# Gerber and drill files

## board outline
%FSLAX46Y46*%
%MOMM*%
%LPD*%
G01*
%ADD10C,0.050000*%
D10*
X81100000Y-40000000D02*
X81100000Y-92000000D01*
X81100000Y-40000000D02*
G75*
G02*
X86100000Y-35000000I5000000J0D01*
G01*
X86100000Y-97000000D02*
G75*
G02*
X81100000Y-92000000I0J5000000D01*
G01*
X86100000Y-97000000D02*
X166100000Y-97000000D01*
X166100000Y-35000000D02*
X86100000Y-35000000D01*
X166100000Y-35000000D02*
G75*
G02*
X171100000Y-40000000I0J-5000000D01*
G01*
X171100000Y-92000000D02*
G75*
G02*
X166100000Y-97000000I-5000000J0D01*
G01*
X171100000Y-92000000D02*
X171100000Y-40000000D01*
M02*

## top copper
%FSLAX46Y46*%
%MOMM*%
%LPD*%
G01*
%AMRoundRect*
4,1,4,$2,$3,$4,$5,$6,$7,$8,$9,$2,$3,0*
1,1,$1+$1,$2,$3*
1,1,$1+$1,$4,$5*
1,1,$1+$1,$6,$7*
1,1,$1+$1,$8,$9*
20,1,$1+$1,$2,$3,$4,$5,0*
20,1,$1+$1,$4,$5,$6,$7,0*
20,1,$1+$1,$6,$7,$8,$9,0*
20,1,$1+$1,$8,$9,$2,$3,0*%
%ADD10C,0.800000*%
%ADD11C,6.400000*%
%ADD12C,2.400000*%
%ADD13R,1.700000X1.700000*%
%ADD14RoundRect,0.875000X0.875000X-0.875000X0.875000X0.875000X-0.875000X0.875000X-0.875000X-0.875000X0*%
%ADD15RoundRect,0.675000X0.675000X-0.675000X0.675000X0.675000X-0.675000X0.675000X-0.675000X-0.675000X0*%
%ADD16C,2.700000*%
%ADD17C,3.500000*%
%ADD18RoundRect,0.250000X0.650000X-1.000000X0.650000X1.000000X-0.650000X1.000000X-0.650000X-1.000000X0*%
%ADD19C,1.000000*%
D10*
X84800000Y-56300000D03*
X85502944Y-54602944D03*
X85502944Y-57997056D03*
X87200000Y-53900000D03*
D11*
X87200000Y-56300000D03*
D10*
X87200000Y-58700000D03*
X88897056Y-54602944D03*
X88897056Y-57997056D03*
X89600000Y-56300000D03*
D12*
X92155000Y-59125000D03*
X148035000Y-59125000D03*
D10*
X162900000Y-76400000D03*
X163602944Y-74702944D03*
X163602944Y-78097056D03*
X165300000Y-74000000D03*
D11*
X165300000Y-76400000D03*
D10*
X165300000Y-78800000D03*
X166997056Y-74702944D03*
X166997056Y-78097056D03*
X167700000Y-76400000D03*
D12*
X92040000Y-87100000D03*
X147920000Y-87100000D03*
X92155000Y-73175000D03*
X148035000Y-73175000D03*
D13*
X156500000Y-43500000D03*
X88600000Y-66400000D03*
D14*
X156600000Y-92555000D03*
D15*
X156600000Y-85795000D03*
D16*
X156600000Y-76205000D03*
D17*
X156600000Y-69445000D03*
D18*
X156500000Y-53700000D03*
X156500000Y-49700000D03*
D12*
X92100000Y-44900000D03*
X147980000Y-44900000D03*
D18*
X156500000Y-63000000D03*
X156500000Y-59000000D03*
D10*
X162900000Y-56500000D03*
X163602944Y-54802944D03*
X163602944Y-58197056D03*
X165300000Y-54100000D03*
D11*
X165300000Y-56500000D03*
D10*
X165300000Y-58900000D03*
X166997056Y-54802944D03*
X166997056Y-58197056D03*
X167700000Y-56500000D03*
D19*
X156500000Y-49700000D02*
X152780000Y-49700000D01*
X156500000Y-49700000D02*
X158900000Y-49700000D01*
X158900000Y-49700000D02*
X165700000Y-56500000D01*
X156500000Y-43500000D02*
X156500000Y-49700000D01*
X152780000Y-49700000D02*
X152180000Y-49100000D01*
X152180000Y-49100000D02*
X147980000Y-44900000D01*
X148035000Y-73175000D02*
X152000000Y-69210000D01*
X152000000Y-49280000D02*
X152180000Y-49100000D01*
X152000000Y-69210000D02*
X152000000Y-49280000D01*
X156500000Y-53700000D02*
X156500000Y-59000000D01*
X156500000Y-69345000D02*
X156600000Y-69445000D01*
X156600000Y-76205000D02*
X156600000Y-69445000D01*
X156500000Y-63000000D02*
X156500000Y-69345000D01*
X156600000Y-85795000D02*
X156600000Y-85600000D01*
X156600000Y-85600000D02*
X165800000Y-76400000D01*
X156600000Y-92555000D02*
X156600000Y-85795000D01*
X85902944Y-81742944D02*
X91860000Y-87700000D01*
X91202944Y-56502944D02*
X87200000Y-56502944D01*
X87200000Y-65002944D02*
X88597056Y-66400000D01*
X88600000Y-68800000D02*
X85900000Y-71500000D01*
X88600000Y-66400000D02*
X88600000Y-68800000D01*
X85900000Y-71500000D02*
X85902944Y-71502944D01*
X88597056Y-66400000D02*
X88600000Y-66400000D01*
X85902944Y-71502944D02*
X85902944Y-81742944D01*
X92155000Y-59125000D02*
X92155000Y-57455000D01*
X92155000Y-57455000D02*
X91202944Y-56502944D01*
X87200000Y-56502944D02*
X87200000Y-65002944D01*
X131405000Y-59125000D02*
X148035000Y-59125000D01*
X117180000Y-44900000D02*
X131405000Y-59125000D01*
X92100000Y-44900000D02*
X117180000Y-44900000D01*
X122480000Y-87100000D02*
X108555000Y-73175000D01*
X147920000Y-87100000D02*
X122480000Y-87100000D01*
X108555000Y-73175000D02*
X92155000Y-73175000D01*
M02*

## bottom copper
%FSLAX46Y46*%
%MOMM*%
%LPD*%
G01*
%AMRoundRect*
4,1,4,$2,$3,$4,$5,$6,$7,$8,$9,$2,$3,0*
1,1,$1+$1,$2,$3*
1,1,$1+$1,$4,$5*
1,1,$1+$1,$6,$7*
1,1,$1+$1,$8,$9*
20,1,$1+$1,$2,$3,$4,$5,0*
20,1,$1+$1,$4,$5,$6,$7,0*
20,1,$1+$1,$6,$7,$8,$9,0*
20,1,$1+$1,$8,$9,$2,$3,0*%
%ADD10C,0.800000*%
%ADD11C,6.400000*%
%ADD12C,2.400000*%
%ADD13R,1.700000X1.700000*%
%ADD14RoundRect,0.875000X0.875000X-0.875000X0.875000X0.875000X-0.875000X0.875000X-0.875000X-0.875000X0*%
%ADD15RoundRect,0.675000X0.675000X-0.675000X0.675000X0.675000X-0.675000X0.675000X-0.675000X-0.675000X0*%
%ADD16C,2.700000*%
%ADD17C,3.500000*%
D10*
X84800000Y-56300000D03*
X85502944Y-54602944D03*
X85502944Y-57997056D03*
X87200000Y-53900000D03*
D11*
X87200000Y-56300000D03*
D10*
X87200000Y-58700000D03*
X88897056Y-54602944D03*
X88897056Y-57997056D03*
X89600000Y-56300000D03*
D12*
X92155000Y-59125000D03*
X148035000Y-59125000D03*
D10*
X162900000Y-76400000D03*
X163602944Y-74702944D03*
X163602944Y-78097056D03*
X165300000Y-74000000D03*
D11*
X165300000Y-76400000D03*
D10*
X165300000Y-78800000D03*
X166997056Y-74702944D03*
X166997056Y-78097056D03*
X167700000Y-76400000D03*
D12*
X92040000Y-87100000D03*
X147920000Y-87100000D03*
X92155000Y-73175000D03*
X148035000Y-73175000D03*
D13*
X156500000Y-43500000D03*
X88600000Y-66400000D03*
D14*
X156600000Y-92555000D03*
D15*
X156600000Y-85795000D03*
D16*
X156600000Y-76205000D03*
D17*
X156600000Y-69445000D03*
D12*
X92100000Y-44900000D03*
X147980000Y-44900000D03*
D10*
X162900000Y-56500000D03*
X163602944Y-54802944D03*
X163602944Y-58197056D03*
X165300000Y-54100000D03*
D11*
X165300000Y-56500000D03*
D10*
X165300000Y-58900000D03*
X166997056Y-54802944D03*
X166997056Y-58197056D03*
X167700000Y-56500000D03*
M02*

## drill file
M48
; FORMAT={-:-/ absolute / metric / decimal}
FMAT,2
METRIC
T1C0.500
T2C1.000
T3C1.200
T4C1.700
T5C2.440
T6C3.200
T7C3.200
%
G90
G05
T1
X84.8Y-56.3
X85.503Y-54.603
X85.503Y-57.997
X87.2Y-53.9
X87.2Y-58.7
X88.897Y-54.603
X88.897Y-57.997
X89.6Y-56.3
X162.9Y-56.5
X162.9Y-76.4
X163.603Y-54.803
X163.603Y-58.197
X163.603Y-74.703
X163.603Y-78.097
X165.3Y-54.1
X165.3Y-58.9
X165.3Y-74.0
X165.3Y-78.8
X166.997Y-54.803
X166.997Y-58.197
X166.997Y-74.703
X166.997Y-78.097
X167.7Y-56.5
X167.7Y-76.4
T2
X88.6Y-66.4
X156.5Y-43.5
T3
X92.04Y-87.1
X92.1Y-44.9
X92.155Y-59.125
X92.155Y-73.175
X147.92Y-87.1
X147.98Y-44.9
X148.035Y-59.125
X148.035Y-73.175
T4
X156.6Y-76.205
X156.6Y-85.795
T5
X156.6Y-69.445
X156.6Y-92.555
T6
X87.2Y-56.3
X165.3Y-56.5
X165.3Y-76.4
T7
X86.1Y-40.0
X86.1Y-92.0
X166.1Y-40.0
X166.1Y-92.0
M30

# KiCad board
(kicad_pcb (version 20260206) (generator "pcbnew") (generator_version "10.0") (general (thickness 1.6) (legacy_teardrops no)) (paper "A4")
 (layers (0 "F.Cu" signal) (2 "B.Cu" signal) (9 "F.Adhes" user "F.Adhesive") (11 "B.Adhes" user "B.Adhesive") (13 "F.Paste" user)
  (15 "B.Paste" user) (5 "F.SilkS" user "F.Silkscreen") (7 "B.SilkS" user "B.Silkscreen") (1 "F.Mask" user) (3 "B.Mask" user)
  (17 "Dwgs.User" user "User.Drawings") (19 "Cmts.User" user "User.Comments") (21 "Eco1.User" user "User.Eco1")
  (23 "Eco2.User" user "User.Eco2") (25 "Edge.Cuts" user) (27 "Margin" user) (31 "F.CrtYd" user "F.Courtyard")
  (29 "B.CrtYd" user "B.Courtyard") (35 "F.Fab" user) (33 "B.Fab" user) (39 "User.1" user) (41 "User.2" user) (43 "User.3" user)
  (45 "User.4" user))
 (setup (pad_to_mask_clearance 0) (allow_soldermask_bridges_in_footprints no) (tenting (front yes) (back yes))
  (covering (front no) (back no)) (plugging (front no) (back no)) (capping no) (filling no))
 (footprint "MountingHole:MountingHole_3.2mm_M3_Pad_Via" (layer "F.Cu") (at 87.2 56.3)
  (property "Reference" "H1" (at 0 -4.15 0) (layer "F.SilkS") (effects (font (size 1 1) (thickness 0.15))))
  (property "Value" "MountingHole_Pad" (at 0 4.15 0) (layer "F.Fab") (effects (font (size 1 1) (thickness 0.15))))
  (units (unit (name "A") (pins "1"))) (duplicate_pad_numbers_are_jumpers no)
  (pad "1" thru_hole circle (at -2.4 0) (size 0.8 0.8) (drill 0.5) (layers "*.Cu" "*.Mask") (remove_unused_layers no) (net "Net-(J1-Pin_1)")
   (zone_connect 2))
  (pad "1" thru_hole circle (at -1.697056 -1.697056) (size 0.8 0.8) (drill 0.5) (layers "*.Cu" "*.Mask") (remove_unused_layers no)
   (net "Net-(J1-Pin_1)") (zone_connect 2))
  (pad "1" thru_hole circle (at -1.697056 1.697056) (size 0.8 0.8) (drill 0.5) (layers "*.Cu" "*.Mask") (remove_unused_layers no)
   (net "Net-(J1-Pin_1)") (zone_connect 2))
  (pad "1" thru_hole circle (at 0 -2.4) (size 0.8 0.8) (drill 0.5) (layers "*.Cu" "*.Mask") (remove_unused_layers no) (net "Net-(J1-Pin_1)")
   (zone_connect 2))
  (pad "1" thru_hole circle (at 0 0) (size 6.4 6.4) (drill 3.2) (layers "*.Cu" "*.Mask") (remove_unused_layers no) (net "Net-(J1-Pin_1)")
   (zone_connect 2))
  (pad "1" thru_hole circle (at 0 2.4) (size 0.8 0.8) (drill 0.5) (layers "*.Cu" "*.Mask") (remove_unused_layers no) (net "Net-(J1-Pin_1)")
   (zone_connect 2))
  (pad "1" thru_hole circle (at 1.697056 -1.697056) (size 0.8 0.8) (drill 0.5) (layers "*.Cu" "*.Mask") (remove_unused_layers no)
   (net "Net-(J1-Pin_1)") (zone_connect 2))
  (pad "1" thru_hole circle (at 1.697056 1.697056) (size 0.8 0.8) (drill 0.5) (layers "*.Cu" "*.Mask") (remove_unused_layers no)
   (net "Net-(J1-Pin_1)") (zone_connect 2))
  (pad "1" thru_hole circle (at 2.4 0) (size 0.8 0.8) (drill 0.5) (layers "*.Cu" "*.Mask") (remove_unused_layers no) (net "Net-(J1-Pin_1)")
   (zone_connect 2)))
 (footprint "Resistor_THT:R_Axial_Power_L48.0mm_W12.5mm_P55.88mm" (layer "F.Cu") (at 92.155 59.125)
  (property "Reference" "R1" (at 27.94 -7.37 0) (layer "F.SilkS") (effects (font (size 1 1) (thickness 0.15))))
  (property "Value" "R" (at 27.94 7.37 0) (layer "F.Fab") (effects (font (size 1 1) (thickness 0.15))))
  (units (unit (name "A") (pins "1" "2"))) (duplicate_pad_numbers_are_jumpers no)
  (pad "1" thru_hole circle (at 0 0) (size 2.4 2.4) (drill 1.2) (layers "*.Cu" "*.Mask") (remove_unused_layers no) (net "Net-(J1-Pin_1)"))
  (pad "2" thru_hole circle (at 55.88 0) (size 2.4 2.4) (drill 1.2) (layers "*.Cu" "*.Mask") (remove_unused_layers no) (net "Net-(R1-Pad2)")))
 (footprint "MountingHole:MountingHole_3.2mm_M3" (layer "F.Cu") (at 166.1 40)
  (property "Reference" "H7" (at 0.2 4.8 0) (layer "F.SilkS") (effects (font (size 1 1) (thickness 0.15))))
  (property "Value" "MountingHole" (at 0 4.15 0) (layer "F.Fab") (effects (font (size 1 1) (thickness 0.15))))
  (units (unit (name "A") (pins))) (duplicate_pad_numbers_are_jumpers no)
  (pad "" np_thru_hole circle (at 0 0) (size 3.2 3.2) (drill 3.2) (layers "*.Cu" "*.Mask")))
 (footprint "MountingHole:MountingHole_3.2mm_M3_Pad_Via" (layer "F.Cu") (at 165.3 76.4)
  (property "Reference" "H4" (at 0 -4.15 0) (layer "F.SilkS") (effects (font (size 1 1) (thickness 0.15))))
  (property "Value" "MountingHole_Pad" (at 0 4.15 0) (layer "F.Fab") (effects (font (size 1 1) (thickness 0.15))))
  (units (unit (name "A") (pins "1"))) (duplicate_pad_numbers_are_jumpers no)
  (pad "1" thru_hole circle (at -2.4 0) (size 0.8 0.8) (drill 0.5) (layers "*.Cu" "*.Mask") (remove_unused_layers no) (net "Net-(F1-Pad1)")
   (zone_connect 2))
  (pad "1" thru_hole circle (at -1.697056 -1.697056) (size 0.8 0.8) (drill 0.5) (layers "*.Cu" "*.Mask") (remove_unused_layers no)
   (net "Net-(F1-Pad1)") (zone_connect 2))
  (pad "1" thru_hole circle (at -1.697056 1.697056) (size 0.8 0.8) (drill 0.5) (layers "*.Cu" "*.Mask") (remove_unused_layers no)
   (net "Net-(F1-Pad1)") (zone_connect 2))
  (pad "1" thru_hole circle (at 0 -2.4) (size 0.8 0.8) (drill 0.5) (layers "*.Cu" "*.Mask") (remove_unused_layers no) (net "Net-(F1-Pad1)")
   (zone_connect 2))
  (pad "1" thru_hole circle (at 0 0) (size 6.4 6.4) (drill 3.2) (layers "*.Cu" "*.Mask") (remove_unused_layers no) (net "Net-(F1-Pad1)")
   (zone_connect 2))
  (pad "1" thru_hole circle (at 0 2.4) (size 0.8 0.8) (drill 0.5) (layers "*.Cu" "*.Mask") (remove_unused_layers no) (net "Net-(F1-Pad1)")
   (zone_connect 2))
  (pad "1" thru_hole circle (at 1.697056 -1.697056) (size 0.8 0.8) (drill 0.5) (layers "*.Cu" "*.Mask") (remove_unused_layers no)
   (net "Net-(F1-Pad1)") (zone_connect 2))
  (pad "1" thru_hole circle (at 1.697056 1.697056) (size 0.8 0.8) (drill 0.5) (layers "*.Cu" "*.Mask") (remove_unused_layers no)
   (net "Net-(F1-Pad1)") (zone_connect 2))
  (pad "1" thru_hole circle (at 2.4 0) (size 0.8 0.8) (drill 0.5) (layers "*.Cu" "*.Mask") (remove_unused_layers no) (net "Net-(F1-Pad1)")
   (zone_connect 2)))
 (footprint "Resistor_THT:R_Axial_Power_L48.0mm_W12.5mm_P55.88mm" (layer "F.Cu") (at 92.04 87.1)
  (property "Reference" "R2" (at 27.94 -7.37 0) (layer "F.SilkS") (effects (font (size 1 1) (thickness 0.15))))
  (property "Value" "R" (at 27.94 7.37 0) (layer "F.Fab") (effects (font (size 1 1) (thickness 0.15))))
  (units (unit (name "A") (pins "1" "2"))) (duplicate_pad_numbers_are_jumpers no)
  (pad "1" thru_hole circle (at 0 0) (size 2.4 2.4) (drill 1.2) (layers "*.Cu" "*.Mask") (remove_unused_layers no) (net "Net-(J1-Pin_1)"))
  (pad "2" thru_hole circle (at 55.88 0) (size 2.4 2.4) (drill 1.2) (layers "*.Cu" "*.Mask") (remove_unused_layers no) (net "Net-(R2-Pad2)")))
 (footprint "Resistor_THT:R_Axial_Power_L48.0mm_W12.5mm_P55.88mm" (layer "F.Cu") (at 92.155 73.175)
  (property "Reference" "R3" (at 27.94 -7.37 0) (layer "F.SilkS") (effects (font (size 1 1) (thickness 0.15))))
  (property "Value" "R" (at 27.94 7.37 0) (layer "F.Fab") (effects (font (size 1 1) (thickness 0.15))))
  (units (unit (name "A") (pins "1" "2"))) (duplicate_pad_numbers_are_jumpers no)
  (pad "1" thru_hole circle (at 0 0) (size 2.4 2.4) (drill 1.2) (layers "*.Cu" "*.Mask") (remove_unused_layers no) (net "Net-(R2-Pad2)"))
  (pad "2" thru_hole circle (at 55.88 0) (size 2.4 2.4) (drill 1.2) (layers "*.Cu" "*.Mask") (remove_unused_layers no) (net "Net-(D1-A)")))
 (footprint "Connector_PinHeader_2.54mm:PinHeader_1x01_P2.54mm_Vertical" (layer "F.Cu") (at 156.5 43.5)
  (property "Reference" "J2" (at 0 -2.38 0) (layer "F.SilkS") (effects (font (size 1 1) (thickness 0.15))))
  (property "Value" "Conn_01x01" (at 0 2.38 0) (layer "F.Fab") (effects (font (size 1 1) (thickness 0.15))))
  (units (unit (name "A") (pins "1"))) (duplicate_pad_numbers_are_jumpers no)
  (pad "1" thru_hole rect (at 0 0) (size 1.7 1.7) (drill 1) (layers "*.Cu" "*.Mask") (remove_unused_layers no) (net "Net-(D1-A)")))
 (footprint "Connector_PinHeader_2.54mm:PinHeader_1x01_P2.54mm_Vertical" (layer "F.Cu") (at 88.6 66.4)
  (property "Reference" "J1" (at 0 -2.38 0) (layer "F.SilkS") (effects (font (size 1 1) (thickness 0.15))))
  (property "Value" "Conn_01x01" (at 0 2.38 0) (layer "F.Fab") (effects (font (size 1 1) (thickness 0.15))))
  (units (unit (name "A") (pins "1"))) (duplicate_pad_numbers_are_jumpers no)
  (pad "1" thru_hole rect (at 0 0) (size 1.7 1.7) (drill 1) (layers "*.Cu" "*.Mask") (remove_unused_layers no) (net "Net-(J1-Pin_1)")))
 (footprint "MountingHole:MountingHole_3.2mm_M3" (layer "F.Cu") (at 86.1 40)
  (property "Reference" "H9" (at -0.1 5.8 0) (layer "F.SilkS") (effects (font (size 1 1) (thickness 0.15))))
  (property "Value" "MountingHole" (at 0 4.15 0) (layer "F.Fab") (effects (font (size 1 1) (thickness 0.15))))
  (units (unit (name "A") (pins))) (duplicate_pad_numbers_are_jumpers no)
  (pad "" np_thru_hole circle (at 0 0) (size 3.2 3.2) (drill 3.2) (layers "*.Cu" "*.Mask")))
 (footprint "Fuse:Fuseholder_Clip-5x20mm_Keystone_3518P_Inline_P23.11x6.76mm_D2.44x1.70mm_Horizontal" (layer "F.Cu") (at 156.6 92.555 90)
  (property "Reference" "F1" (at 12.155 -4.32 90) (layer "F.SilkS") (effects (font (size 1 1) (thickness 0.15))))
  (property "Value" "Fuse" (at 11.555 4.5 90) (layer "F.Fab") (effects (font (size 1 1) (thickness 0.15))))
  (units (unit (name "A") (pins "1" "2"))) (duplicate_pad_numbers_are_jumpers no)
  (pad "1" thru_hole roundrect (at 0 0 90) (size 3.5 3.5) (drill 2.44) (layers "*.Cu" "*.Mask") (remove_unused_layers no)
   (roundrect_rratio 0.25) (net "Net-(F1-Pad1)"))
  (pad "1" thru_hole roundrect (at 6.76 0 90) (size 2.7 2.7) (drill 1.7) (layers "*.Cu" "*.Mask") (remove_unused_layers no)
   (roundrect_rratio 0.25) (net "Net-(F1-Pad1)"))
  (pad "2" thru_hole circle (at 16.35 0 90) (size 2.7 2.7) (drill 1.7) (layers "*.Cu" "*.Mask") (remove_unused_layers no) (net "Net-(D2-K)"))
  (pad "2" thru_hole circle (at 23.11 0 90) (size 3.5 3.5) (drill 2.44) (layers "*.Cu" "*.Mask") (remove_unused_layers no)
   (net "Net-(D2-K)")))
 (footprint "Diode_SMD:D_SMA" (layer "F.Cu") (at 156.5 51.7 90)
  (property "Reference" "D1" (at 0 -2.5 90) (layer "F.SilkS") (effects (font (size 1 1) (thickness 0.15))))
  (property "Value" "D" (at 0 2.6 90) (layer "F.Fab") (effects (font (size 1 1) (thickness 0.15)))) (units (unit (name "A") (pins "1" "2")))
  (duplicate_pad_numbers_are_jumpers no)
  (pad "1" smd roundrect (at -2 0 90) (size 2.5 1.8) (layers "F.Cu" "F.Mask" "F.Paste") (roundrect_rratio 0.1388888889) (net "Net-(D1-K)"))
  (pad "2" smd roundrect (at 2 0 90) (size 2.5 1.8) (layers "F.Cu" "F.Mask" "F.Paste") (roundrect_rratio 0.1388888889) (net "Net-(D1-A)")))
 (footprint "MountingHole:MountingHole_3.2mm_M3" (layer "F.Cu") (at 86.1 92)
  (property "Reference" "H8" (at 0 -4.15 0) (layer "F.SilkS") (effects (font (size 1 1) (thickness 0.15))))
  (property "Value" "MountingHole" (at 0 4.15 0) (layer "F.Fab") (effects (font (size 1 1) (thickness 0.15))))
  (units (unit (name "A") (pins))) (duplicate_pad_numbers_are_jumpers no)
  (pad "" np_thru_hole circle (at 0 0) (size 3.2 3.2) (drill 3.2) (layers "*.Cu" "*.Mask")))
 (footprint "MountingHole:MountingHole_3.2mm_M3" (layer "F.Cu") (at 166.1 92)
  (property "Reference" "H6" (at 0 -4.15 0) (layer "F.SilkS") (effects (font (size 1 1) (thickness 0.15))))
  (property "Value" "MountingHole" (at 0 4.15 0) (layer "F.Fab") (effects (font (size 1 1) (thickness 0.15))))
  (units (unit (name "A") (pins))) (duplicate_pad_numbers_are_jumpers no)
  (pad "" np_thru_hole circle (at 0 0) (size 3.2 3.2) (drill 3.2) (layers "*.Cu" "*.Mask")))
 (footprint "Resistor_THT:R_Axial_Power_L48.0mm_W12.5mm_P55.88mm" (layer "F.Cu") (at 92.1 44.9)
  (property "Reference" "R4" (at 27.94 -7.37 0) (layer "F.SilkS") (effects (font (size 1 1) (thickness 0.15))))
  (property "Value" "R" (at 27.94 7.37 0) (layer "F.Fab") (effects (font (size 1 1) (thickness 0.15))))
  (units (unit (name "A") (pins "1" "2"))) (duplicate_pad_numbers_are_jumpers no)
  (pad "1" thru_hole circle (at 0 0) (size 2.4 2.4) (drill 1.2) (layers "*.Cu" "*.Mask") (remove_unused_layers no) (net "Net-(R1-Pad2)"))
  (pad "2" thru_hole circle (at 55.88 0) (size 2.4 2.4) (drill 1.2) (layers "*.Cu" "*.Mask") (remove_unused_layers no) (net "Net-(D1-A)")))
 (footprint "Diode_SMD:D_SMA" (layer "F.Cu") (at 156.5 61 90)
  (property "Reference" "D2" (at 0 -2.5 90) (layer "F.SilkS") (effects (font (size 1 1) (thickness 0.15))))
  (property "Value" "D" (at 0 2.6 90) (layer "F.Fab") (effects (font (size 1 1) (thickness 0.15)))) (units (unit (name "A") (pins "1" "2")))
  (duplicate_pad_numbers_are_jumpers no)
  (pad "1" smd roundrect (at -2 0 90) (size 2.5 1.8) (layers "F.Cu" "F.Mask" "F.Paste") (roundrect_rratio 0.1388888889) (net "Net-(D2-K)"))
  (pad "2" smd roundrect (at 2 0 90) (size 2.5 1.8) (layers "F.Cu" "F.Mask" "F.Paste") (roundrect_rratio 0.1388888889) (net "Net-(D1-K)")))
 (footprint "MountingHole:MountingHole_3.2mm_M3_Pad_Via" (layer "F.Cu") (at 165.3 56.5)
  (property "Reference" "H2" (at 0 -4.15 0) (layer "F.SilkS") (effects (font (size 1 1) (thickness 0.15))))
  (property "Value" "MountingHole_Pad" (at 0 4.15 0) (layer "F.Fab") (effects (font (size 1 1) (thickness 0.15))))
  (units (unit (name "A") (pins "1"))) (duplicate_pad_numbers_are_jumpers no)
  (pad "1" thru_hole circle (at -2.4 0) (size 0.8 0.8) (drill 0.5) (layers "*.Cu" "*.Mask") (remove_unused_layers no) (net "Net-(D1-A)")
   (zone_connect 2))
  (pad "1" thru_hole circle (at -1.697056 -1.697056) (size 0.8 0.8) (drill 0.5) (layers "*.Cu" "*.Mask") (remove_unused_layers no)
   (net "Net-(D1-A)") (zone_connect 2))
  (pad "1" thru_hole circle (at -1.697056 1.697056) (size 0.8 0.8) (drill 0.5) (layers "*.Cu" "*.Mask") (remove_unused_layers no)
   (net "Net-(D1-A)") (zone_connect 2))
  (pad "1" thru_hole circle (at 0 -2.4) (size 0.8 0.8) (drill 0.5) (layers "*.Cu" "*.Mask") (remove_unused_layers no) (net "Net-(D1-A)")
   (zone_connect 2))
  (pad "1" thru_hole circle (at 0 0) (size 6.4 6.4) (drill 3.2) (layers "*.Cu" "*.Mask") (remove_unused_layers no) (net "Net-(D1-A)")
   (zone_connect 2))
  (pad "1" thru_hole circle (at 0 2.4) (size 0.8 0.8) (drill 0.5) (layers "*.Cu" "*.Mask") (remove_unused_layers no) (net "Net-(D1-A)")
   (zone_connect 2))
  (pad "1" thru_hole circle (at 1.697056 -1.697056) (size 0.8 0.8) (drill 0.5) (layers "*.Cu" "*.Mask") (remove_unused_layers no)
   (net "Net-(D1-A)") (zone_connect 2))
  (pad "1" thru_hole circle (at 1.697056 1.697056) (size 0.8 0.8) (drill 0.5) (layers "*.Cu" "*.Mask") (remove_unused_layers no)
   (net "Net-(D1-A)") (zone_connect 2))
  (pad "1" thru_hole circle (at 2.4 0) (size 0.8 0.8) (drill 0.5) (layers "*.Cu" "*.Mask") (remove_unused_layers no) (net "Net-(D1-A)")
   (zone_connect 2)))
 (gr_line (start 81.1 40) (end 81.1 92) (stroke (width 0.05) (type default)) (layer "Edge.Cuts"))
 (gr_arc (start 81.1 40) (mid 82.564466 36.464466) (end 86.1 35) (stroke (width 0.05) (type default)) (layer "Edge.Cuts"))
 (gr_arc (start 86.1 97) (mid 82.564466 95.535534) (end 81.1 92) (stroke (width 0.05) (type default)) (layer "Edge.Cuts"))
 (gr_line (start 86.1 97) (end 166.1 97) (stroke (width 0.05) (type default)) (layer "Edge.Cuts"))
 (gr_line (start 166.1 35) (end 86.1 35) (stroke (width 0.05) (type default)) (layer "Edge.Cuts"))
 (gr_arc (start 166.1 35) (mid 169.635534 36.464466) (end 171.1 40) (stroke (width 0.05) (type default)) (layer "Edge.Cuts"))
 (gr_arc (start 171.1 92) (mid 169.635534 95.535534) (end 166.1 97) (stroke (width 0.05) (type default)) (layer "Edge.Cuts"))
 (gr_line (start 171.1 92) (end 171.1 40) (stroke (width 0.05) (type default)) (layer "Edge.Cuts"))
 (segment (start 156.5 49.7) (end 152.78 49.7) (width 1) (layer "F.Cu") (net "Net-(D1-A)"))
 (segment (start 156.5 49.7) (end 158.9 49.7) (width 1) (layer "F.Cu") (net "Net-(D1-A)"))
 (segment (start 158.9 49.7) (end 165.7 56.5) (width 1) (layer "F.Cu") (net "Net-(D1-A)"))
 (segment (start 156.5 43.5) (end 156.5 49.7) (width 1) (layer "F.Cu") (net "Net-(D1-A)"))
 (segment (start 152.78 49.7) (end 152.18 49.1) (width 1) (layer "F.Cu") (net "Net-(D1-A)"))
 (segment (start 152.18 49.1) (end 147.98 44.9) (width 1) (layer "F.Cu") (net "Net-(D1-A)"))
 (segment (start 148.035 73.175) (end 152 69.21) (width 1) (layer "F.Cu") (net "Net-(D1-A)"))
 (segment (start 152 49.28) (end 152.18 49.1) (width 1) (layer "F.Cu") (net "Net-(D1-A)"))
 (segment (start 152 69.21) (end 152 49.28) (width 1) (layer "F.Cu") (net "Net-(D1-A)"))
 (segment (start 156.5 53.7) (end 156.5 59) (width 1) (layer "F.Cu") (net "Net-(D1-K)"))
 (segment (start 156.5 69.345) (end 156.6 69.445) (width 1) (layer "F.Cu") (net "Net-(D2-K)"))
 (segment (start 156.6 76.205) (end 156.6 69.445) (width 1) (layer "F.Cu") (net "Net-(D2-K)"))
 (segment (start 156.5 63) (end 156.5 69.345) (width 1) (layer "F.Cu") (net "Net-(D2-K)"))
 (segment (start 156.6 85.795) (end 156.6 85.6) (width 1) (layer "F.Cu") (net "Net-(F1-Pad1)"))
 (segment (start 156.6 85.6) (end 165.8 76.4) (width 1) (layer "F.Cu") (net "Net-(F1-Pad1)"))
 (segment (start 156.6 92.555) (end 156.6 85.795) (width 1) (layer "F.Cu") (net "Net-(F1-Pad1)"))
 (segment (start 85.902944 81.742944) (end 91.86 87.7) (width 1) (layer "F.Cu") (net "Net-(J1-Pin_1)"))
 (segment (start 91.202944 56.502944) (end 87.2 56.502944) (width 1) (layer "F.Cu") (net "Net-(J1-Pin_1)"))
 (segment (start 87.2 65.002944) (end 88.597056 66.4) (width 1) (layer "F.Cu") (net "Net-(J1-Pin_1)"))
 (segment (start 88.6 68.8) (end 85.9 71.5) (width 1) (layer "F.Cu") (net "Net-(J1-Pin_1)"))
 (segment (start 88.6 66.4) (end 88.6 68.8) (width 1) (layer "F.Cu") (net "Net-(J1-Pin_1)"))
 (segment (start 85.9 71.5) (end 85.902944 71.502944) (width 1) (layer "F.Cu") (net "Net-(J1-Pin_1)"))
 (segment (start 88.597056 66.4) (end 88.6 66.4) (width 1) (layer "F.Cu") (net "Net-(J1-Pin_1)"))
 (segment (start 85.902944 71.502944) (end 85.902944 81.742944) (width 1) (layer "F.Cu") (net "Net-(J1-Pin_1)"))
 (segment (start 92.155 59.125) (end 92.155 57.455) (width 1) (layer "F.Cu") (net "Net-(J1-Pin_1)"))
 (segment (start 92.155 57.455) (end 91.202944 56.502944) (width 1) (layer "F.Cu") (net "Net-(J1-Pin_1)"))
 (segment (start 87.2 56.502944) (end 87.2 65.002944) (width 1) (layer "F.Cu") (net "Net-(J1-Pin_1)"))
 (segment (start 131.405 59.125) (end 148.035 59.125) (width 1) (layer "F.Cu") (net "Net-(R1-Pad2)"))
 (segment (start 117.18 44.9) (end 131.405 59.125) (width 1) (layer "F.Cu") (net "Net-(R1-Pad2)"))
 (segment (start 92.1 44.9) (end 117.18 44.9) (width 1) (layer "F.Cu") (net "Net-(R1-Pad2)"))
 (segment (start 122.48 87.1) (end 108.555 73.175) (width 1) (layer "F.Cu") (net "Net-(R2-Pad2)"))
 (segment (start 147.92 87.1) (end 122.48 87.1) (width 1) (layer "F.Cu") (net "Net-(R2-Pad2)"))
 (segment (start 108.555 73.175) (end 92.155 73.175) (width 1) (layer "F.Cu") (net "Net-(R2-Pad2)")))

